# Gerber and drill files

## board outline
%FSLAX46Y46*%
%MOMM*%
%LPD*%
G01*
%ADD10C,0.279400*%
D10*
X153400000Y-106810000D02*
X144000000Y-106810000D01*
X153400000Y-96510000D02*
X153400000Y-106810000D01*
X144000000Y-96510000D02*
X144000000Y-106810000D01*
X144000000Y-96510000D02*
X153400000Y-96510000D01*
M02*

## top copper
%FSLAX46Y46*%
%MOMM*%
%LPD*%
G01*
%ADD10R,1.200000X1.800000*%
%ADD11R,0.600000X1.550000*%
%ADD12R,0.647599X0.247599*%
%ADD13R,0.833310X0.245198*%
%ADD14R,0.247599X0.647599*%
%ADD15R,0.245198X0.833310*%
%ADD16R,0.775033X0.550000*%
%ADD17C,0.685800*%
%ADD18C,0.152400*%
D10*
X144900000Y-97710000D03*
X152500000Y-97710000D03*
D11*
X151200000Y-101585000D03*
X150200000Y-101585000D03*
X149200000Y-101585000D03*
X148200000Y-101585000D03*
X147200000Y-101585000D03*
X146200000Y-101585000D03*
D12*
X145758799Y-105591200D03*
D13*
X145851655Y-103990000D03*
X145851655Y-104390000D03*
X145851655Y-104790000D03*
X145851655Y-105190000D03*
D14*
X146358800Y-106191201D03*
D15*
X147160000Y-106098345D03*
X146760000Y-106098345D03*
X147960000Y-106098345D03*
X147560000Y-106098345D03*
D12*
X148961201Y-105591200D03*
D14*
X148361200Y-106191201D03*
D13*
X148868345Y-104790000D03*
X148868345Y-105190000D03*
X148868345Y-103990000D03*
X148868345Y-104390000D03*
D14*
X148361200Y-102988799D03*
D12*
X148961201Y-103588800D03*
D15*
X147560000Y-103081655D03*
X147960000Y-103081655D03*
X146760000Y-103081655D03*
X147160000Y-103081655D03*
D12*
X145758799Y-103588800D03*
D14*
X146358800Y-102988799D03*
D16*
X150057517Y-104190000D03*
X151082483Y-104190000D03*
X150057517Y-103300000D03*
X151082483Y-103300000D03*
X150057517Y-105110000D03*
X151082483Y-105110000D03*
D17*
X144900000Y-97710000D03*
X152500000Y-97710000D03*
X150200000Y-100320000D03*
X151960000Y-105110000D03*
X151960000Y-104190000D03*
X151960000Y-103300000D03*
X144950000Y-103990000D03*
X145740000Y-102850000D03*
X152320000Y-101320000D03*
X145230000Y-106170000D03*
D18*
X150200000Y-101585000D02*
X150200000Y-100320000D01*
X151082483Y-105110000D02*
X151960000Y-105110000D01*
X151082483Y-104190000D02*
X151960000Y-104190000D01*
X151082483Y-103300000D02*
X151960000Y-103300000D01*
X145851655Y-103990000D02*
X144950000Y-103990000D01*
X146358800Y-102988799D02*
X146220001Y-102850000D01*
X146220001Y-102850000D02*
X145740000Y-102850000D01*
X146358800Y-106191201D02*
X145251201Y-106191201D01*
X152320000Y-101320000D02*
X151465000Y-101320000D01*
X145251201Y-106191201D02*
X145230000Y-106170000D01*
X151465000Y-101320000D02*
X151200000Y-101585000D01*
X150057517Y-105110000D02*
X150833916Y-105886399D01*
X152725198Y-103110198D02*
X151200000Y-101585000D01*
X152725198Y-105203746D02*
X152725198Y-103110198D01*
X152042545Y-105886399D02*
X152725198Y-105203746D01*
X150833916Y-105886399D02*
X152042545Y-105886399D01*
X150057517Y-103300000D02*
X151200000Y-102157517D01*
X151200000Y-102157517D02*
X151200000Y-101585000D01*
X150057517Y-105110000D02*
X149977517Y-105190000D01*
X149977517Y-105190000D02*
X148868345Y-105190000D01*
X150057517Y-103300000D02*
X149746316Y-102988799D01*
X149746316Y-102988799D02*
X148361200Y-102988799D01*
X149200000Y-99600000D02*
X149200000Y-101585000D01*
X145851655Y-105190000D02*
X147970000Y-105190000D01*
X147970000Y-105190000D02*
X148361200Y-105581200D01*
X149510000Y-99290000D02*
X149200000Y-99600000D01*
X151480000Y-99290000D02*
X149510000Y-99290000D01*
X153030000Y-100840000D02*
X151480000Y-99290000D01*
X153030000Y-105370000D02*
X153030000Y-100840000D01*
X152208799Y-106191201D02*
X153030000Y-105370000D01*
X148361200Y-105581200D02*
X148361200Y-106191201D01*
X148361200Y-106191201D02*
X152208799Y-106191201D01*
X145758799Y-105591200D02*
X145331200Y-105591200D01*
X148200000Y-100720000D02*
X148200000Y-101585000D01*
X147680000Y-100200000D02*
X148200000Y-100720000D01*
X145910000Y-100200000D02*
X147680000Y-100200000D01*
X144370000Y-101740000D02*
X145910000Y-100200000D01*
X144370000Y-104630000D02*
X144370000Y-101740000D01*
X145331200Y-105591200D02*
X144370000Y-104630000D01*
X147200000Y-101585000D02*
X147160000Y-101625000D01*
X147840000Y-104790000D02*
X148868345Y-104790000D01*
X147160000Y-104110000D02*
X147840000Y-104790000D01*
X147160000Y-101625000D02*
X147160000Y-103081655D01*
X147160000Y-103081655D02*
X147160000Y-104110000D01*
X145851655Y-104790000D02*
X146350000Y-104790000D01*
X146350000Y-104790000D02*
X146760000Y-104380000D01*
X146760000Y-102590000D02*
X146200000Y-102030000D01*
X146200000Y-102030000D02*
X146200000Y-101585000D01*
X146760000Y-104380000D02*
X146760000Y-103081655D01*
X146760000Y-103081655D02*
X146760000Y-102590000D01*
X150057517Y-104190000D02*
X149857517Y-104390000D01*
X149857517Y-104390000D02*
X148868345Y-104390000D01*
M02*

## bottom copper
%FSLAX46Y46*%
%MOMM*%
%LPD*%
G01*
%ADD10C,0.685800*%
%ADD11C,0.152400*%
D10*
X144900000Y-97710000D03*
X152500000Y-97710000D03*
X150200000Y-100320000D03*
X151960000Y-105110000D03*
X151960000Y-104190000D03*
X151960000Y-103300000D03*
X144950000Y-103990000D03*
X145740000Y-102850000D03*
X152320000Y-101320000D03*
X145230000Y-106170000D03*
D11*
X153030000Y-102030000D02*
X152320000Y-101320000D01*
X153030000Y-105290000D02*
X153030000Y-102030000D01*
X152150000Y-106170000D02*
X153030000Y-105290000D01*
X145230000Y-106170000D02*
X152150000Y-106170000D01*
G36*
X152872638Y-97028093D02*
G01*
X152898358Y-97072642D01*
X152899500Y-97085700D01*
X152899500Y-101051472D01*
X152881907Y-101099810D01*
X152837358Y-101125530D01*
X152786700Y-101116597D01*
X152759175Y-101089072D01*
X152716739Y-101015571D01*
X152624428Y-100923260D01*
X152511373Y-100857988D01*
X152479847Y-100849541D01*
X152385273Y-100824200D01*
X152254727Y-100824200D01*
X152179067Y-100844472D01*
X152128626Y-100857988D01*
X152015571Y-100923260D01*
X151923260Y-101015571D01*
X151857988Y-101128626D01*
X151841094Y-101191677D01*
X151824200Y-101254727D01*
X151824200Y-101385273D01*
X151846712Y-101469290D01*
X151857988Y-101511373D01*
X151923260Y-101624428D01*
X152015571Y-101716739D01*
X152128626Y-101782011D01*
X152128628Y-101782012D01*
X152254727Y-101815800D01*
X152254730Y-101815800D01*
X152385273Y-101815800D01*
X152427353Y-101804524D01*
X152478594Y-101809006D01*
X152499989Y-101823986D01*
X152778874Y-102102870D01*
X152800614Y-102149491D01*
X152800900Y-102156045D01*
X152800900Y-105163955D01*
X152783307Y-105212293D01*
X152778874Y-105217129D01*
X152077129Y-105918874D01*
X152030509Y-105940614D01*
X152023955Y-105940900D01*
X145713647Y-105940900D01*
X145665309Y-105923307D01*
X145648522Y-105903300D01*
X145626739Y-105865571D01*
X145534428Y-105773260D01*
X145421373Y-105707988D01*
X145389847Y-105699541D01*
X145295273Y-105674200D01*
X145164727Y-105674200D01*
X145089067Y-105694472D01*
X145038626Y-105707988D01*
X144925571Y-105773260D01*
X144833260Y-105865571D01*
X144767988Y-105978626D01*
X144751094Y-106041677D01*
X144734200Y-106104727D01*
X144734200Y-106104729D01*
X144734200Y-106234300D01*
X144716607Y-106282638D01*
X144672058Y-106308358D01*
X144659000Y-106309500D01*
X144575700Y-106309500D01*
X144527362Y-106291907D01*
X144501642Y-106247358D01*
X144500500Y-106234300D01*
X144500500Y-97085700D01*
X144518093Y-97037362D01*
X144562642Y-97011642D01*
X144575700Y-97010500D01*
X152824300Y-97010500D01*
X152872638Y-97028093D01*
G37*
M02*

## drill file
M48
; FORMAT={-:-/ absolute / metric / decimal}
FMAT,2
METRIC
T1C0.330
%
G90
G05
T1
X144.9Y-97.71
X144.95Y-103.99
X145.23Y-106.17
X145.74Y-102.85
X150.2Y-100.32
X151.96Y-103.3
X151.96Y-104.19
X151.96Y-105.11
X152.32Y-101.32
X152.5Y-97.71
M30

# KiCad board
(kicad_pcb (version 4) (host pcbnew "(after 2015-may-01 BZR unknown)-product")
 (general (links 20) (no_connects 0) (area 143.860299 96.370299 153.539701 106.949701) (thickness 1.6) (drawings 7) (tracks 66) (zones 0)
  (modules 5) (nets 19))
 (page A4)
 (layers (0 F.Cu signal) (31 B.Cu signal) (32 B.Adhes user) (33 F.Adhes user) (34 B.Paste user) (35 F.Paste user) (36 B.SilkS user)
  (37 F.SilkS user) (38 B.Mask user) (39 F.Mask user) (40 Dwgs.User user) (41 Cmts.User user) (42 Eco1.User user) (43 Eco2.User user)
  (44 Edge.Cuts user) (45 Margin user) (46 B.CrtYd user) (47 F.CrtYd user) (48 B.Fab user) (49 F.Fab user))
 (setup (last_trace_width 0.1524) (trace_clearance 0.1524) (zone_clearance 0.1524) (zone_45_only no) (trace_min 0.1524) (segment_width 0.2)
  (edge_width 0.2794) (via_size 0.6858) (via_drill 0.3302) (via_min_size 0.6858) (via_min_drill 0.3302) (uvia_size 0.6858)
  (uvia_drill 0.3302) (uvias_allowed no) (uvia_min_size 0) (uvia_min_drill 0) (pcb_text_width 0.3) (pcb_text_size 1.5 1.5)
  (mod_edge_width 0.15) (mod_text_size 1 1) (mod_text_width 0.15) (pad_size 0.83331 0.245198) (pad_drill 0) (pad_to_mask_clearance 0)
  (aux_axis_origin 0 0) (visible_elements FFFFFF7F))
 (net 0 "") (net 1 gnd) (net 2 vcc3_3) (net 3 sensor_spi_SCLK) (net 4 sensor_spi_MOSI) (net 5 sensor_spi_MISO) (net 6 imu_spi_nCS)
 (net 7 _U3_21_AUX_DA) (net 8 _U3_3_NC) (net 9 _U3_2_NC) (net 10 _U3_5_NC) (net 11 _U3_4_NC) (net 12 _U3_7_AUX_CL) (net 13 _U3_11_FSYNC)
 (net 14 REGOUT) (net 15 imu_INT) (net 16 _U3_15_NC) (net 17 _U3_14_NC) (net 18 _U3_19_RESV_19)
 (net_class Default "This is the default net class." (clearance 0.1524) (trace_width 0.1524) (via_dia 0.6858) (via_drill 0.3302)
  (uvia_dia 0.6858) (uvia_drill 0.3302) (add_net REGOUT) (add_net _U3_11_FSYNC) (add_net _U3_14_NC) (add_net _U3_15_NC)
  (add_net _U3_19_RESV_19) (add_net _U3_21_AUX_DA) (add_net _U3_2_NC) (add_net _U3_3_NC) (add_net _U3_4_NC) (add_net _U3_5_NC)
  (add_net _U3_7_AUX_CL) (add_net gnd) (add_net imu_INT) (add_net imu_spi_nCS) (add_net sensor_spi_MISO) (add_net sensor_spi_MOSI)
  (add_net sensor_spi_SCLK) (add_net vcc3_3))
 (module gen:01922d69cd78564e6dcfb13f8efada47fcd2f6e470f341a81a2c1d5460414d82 (layer F.Cu) (at 148.7 96.81)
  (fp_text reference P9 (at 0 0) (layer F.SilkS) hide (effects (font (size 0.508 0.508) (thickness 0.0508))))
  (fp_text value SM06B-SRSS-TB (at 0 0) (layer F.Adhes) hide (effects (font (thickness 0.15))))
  (pad M smd rect (at -3.8 0.9) (size 1.2 1.8) (layers F.Cu F.Paste F.Mask) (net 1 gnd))
  (pad M smd rect (at 3.8 0.9) (size 1.2 1.8) (layers F.Cu F.Paste F.Mask) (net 1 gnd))
  (pad 1 smd rect (at 2.5 4.775) (size 0.6 1.55) (layers F.Cu F.Paste F.Mask) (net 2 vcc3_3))
  (pad 2 smd rect (at 1.5 4.775) (size 0.6 1.55) (layers F.Cu F.Paste F.Mask) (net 1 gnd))
  (pad 3 smd rect (at 0.5 4.775) (size 0.6 1.55) (layers F.Cu F.Paste F.Mask) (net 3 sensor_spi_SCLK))
  (pad 4 smd rect (at -0.5 4.775) (size 0.6 1.55) (layers F.Cu F.Paste F.Mask) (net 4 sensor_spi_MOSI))
  (pad 5 smd rect (at -1.5 4.775) (size 0.6 1.55) (layers F.Cu F.Paste F.Mask) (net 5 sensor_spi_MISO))
  (pad 6 smd rect (at -2.5 4.775) (size 0.6 1.55) (layers F.Cu F.Paste F.Mask) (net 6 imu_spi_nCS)))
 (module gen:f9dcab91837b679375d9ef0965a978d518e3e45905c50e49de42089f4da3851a (layer F.Cu) (at 147.36 104.59 90)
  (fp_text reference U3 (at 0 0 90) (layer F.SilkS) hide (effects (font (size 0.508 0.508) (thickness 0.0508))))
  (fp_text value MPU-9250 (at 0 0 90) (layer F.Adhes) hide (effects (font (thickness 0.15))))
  (pad 24 smd rect (at -1.0012 -1.601201 90) (size 0.247599 0.647599) (layers F.Cu F.Paste F.Mask) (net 4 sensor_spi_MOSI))
  (pad 20 smd rect (at 0.6 -1.508345 90) (size 0.245198 0.83331) (layers F.Cu F.Paste F.Mask) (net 1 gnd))
  (pad 21 smd rect (at 0.2 -1.508345 90) (size 0.245198 0.83331) (layers F.Cu F.Paste F.Mask) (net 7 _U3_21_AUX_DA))
  (pad 22 smd rect (at -0.2 -1.508345 90) (size 0.245198 0.83331) (layers F.Cu F.Paste F.Mask) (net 6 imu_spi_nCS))
  (pad 23 smd rect (at -0.6 -1.508345 90) (size 0.245198 0.83331) (layers F.Cu F.Paste F.Mask) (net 3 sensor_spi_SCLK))
  (pad 1 smd rect (at -1.601201 -1.0012 90) (size 0.647599 0.247599) (layers F.Cu F.Paste F.Mask) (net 2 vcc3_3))
  (pad 3 smd rect (at -1.508345 -0.2 90) (size 0.83331 0.245198) (layers F.Cu F.Paste F.Mask) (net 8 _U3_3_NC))
  (pad 2 smd rect (at -1.508345 -0.6 90) (size 0.83331 0.245198) (layers F.Cu F.Paste F.Mask) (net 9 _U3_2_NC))
  (pad 5 smd rect (at -1.508345 0.6 90) (size 0.83331 0.245198) (layers F.Cu F.Paste F.Mask) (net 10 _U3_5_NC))
  (pad 4 smd rect (at -1.508345 0.2 90) (size 0.83331 0.245198) (layers F.Cu F.Paste F.Mask) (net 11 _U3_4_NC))
  (pad 7 smd rect (at -1.0012 1.601201 90) (size 0.247599 0.647599) (layers F.Cu F.Paste F.Mask) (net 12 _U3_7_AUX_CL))
  (pad 6 smd rect (at -1.601201 1.0012 90) (size 0.647599 0.247599) (layers F.Cu F.Paste F.Mask) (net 3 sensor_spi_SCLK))
  (pad 9 smd rect (at -0.2 1.508345 90) (size 0.245198 0.83331) (layers F.Cu F.Paste F.Mask) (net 5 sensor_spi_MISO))
  (pad 8 smd rect (at -0.6 1.508345 90) (size 0.245198 0.83331) (layers F.Cu F.Paste F.Mask) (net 2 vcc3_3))
  (pad 11 smd rect (at 0.6 1.508345 90) (size 0.245198 0.83331) (layers F.Cu F.Paste F.Mask) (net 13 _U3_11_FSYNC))
  (pad 10 smd rect (at 0.2 1.508345 90) (size 0.245198 0.83331) (layers F.Cu F.Paste F.Mask) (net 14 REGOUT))
  (pad 13 smd rect (at 1.601201 1.0012 90) (size 0.647599 0.247599) (layers F.Cu F.Paste F.Mask) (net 2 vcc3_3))
  (pad 12 smd rect (at 1.0012 1.601201 90) (size 0.247599 0.647599) (layers F.Cu F.Paste F.Mask) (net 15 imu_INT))
  (pad 15 smd rect (at 1.508345 0.2 90) (size 0.83331 0.245198) (layers F.Cu F.Paste F.Mask) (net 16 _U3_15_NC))
  (pad 14 smd rect (at 1.508345 0.6 90) (size 0.83331 0.245198) (layers F.Cu F.Paste F.Mask) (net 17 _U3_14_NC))
  (pad 17 smd rect (at 1.508345 -0.6 90) (size 0.83331 0.245198) (layers F.Cu F.Paste F.Mask) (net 6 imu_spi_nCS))
  (pad 16 smd rect (at 1.508345 -0.2 90) (size 0.83331 0.245198) (layers F.Cu F.Paste F.Mask) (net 5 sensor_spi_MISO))
  (pad 19 smd rect (at 1.0012 -1.601201 90) (size 0.247599 0.647599) (layers F.Cu F.Paste F.Mask) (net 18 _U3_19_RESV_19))
  (pad 18 smd rect (at 1.601201 -1.0012 90) (size 0.647599 0.247599) (layers F.Cu F.Paste F.Mask) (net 1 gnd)))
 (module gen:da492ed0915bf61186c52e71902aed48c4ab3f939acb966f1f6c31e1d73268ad (layer F.Cu) (at 150.57 104.19)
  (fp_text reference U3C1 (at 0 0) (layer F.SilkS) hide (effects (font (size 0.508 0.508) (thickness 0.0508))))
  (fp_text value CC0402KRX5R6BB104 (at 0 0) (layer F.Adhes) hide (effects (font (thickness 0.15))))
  (pad 1 smd rect (at -0.512483 0) (size 0.775033 0.55) (layers F.Cu F.Paste F.Mask) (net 14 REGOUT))
  (pad 2 smd rect (at 0.512483 0) (size 0.775033 0.55) (layers F.Cu F.Paste F.Mask) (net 1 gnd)))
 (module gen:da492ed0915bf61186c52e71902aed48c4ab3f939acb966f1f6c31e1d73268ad (layer F.Cu) (at 150.57 103.3)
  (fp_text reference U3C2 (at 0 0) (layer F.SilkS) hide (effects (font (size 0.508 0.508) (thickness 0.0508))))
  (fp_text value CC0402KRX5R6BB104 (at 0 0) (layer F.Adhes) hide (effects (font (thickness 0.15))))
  (pad 1 smd rect (at -0.512483 0) (size 0.775033 0.55) (layers F.Cu F.Paste F.Mask) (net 2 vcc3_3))
  (pad 2 smd rect (at 0.512483 0) (size 0.775033 0.55) (layers F.Cu F.Paste F.Mask) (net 1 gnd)))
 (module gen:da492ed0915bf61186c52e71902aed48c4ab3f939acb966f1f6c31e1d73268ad (layer F.Cu) (at 150.57 105.11)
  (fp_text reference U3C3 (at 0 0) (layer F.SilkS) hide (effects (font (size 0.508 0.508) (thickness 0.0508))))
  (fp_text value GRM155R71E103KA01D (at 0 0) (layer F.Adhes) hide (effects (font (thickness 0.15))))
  (pad 1 smd rect (at -0.512483 0) (size 0.775033 0.55) (layers F.Cu F.Paste F.Mask) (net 2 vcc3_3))
  (pad 2 smd rect (at 0.512483 0) (size 0.775033 0.55) (layers F.Cu F.Paste F.Mask) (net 1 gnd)))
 (gr_line (start 153.4 106.81) (end 144 106.81) (angle 90) (layer Edge.Cuts) (width 0.2794))
 (gr_line (start 153.4 96.51) (end 153.4 106.81) (angle 90) (layer Edge.Cuts) (width 0.2794))
 (gr_line (start 144 96.51) (end 144 106.81) (angle 90) (layer Edge.Cuts) (width 0.2794))
 (gr_line (start 144 96.51) (end 153.4 96.51) (angle 90) (layer Edge.Cuts) (width 0.2794))
 (via (at 144.9 97.71) (size 0.6858) (layers F.Cu B.Cu) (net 1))
 (via (at 152.5 97.71) (size 0.6858) (layers F.Cu B.Cu) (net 1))
 (segment (start 150.2 101.585) (end 150.2 100.32) (width 0.1524) (layer F.Cu) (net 1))
 (via (at 150.2 100.32) (size 0.6858) (layers F.Cu B.Cu) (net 1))
 (segment (start 151.082483 105.11) (end 151.96 105.11) (width 0.1524) (layer F.Cu) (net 1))
 (via (at 151.96 105.11) (size 0.6858) (layers F.Cu B.Cu) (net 1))
 (segment (start 151.082483 104.19) (end 151.96 104.19) (width 0.1524) (layer F.Cu) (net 1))
 (via (at 151.96 104.19) (size 0.6858) (layers F.Cu B.Cu) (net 1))
 (segment (start 151.082483 103.3) (end 151.96 103.3) (width 0.1524) (layer F.Cu) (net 1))
 (via (at 151.96 103.3) (size 0.6858) (layers F.Cu B.Cu) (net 1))
 (segment (start 145.851655 103.99) (end 144.95 103.99) (width 0.1524) (layer F.Cu) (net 1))
 (via (at 144.95 103.99) (size 0.6858) (layers F.Cu B.Cu) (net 1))
 (segment (start 146.3588 102.988799) (end 146.220001 102.85) (width 0.1524) (layer F.Cu) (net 1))
 (via (at 145.74 102.85) (size 0.6858) (layers F.Cu B.Cu) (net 1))
 (segment (start 146.220001 102.85) (end 145.74 102.85) (width 0.1524) (layer F.Cu) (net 1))
 (segment (start 146.3588 106.191201) (end 145.251201 106.191201) (width 0.1524) (layer F.Cu) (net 2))
 (segment (start 152.32 101.32) (end 151.465 101.32) (width 0.1524) (layer F.Cu) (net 2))
 (via (at 152.32 101.32) (size 0.6858) (layers F.Cu B.Cu) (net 2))
 (segment (start 153.03 102.03) (end 152.32 101.32) (width 0.1524) (layer B.Cu) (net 2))
 (segment (start 153.03 105.29) (end 153.03 102.03) (width 0.1524) (layer B.Cu) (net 2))
 (segment (start 152.15 106.17) (end 153.03 105.29) (width 0.1524) (layer B.Cu) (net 2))
 (segment (start 145.23 106.17) (end 152.15 106.17) (width 0.1524) (layer B.Cu) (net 2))
 (via (at 145.23 106.17) (size 0.6858) (layers F.Cu B.Cu) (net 2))
 (segment (start 145.251201 106.191201) (end 145.23 106.17) (width 0.1524) (layer F.Cu) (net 2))
 (segment (start 151.465 101.32) (end 151.2 101.585) (width 0.1524) (layer F.Cu) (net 2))
 (segment (start 150.057517 105.11) (end 150.833916 105.886399) (width 0.1524) (layer F.Cu) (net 2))
 (segment (start 152.725198 103.110198) (end 151.2 101.585) (width 0.1524) (layer F.Cu) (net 2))
 (segment (start 152.725198 105.203746) (end 152.725198 103.110198) (width 0.1524) (layer F.Cu) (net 2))
 (segment (start 152.042545 105.886399) (end 152.725198 105.203746) (width 0.1524) (layer F.Cu) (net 2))
 (segment (start 150.833916 105.886399) (end 152.042545 105.886399) (width 0.1524) (layer F.Cu) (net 2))
 (segment (start 150.057517 103.3) (end 151.2 102.157517) (width 0.1524) (layer F.Cu) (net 2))
 (segment (start 151.2 102.157517) (end 151.2 101.585) (width 0.1524) (layer F.Cu) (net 2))
 (segment (start 150.057517 105.11) (end 149.977517 105.19) (width 0.1524) (layer F.Cu) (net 2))
 (segment (start 149.977517 105.19) (end 148.868345 105.19) (width 0.1524) (layer F.Cu) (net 2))
 (segment (start 150.057517 103.3) (end 149.746316 102.988799) (width 0.1524) (layer F.Cu) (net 2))
 (segment (start 149.746316 102.988799) (end 148.3612 102.988799) (width 0.1524) (layer F.Cu) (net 2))
 (segment (start 149.2 99.6) (end 149.2 101.585) (width 0.1524) (layer F.Cu) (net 3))
 (segment (start 145.851655 105.19) (end 147.97 105.19) (width 0.1524) (layer F.Cu) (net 3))
 (segment (start 147.97 105.19) (end 148.3612 105.5812) (width 0.1524) (layer F.Cu) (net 3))
 (segment (start 149.51 99.29) (end 149.2 99.6) (width 0.1524) (layer F.Cu) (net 3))
 (segment (start 151.48 99.29) (end 149.51 99.29) (width 0.1524) (layer F.Cu) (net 3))
 (segment (start 153.03 100.84) (end 151.48 99.29) (width 0.1524) (layer F.Cu) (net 3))
 (segment (start 153.03 105.37) (end 153.03 100.84) (width 0.1524) (layer F.Cu) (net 3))
 (segment (start 152.208799 106.191201) (end 153.03 105.37) (width 0.1524) (layer F.Cu) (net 3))
 (segment (start 148.3612 105.5812) (end 148.3612 106.191201) (width 0.1524) (layer F.Cu) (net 3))
 (segment (start 148.3612 106.191201) (end 152.208799 106.191201) (width 0.1524) (layer F.Cu) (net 3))
 (segment (start 145.758799 105.5912) (end 145.3312 105.5912) (width 0.1524) (layer F.Cu) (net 4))
 (segment (start 148.2 100.72) (end 148.2 101.585) (width 0.1524) (layer F.Cu) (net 4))
 (segment (start 147.68 100.2) (end 148.2 100.72) (width 0.1524) (layer F.Cu) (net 4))
 (segment (start 145.91 100.2) (end 147.68 100.2) (width 0.1524) (layer F.Cu) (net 4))
 (segment (start 144.37 101.74) (end 145.91 100.2) (width 0.1524) (layer F.Cu) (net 4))
 (segment (start 144.37 104.63) (end 144.37 101.74) (width 0.1524) (layer F.Cu) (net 4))
 (segment (start 145.3312 105.5912) (end 144.37 104.63) (width 0.1524) (layer F.Cu) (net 4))
 (segment (start 147.2 101.585) (end 147.16 101.625) (width 0.1524) (layer F.Cu) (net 5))
 (segment (start 147.84 104.79) (end 148.868345 104.79) (width 0.1524) (layer F.Cu) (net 5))
 (segment (start 147.16 104.11) (end 147.84 104.79) (width 0.1524) (layer F.Cu) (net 5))
 (segment (start 147.16 101.625) (end 147.16 103.081655) (width 0.1524) (layer F.Cu) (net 5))
 (segment (start 147.16 103.081655) (end 147.16 104.11) (width 0.1524) (layer F.Cu) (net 5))
 (segment (start 145.851655 104.79) (end 146.35 104.79) (width 0.1524) (layer F.Cu) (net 6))
 (segment (start 146.35 104.79) (end 146.76 104.38) (width 0.1524) (layer F.Cu) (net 6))
 (segment (start 146.76 102.59) (end 146.2 102.03) (width 0.1524) (layer F.Cu) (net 6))
 (segment (start 146.2 102.03) (end 146.2 101.585) (width 0.1524) (layer F.Cu) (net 6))
 (segment (start 146.76 104.38) (end 146.76 103.081655) (width 0.1524) (layer F.Cu) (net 6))
 (segment (start 146.76 103.081655) (end 146.76 102.59) (width 0.1524) (layer F.Cu) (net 6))
 (segment (start 150.057517 104.19) (end 149.857517 104.39) (width 0.1524) (layer F.Cu) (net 14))
 (segment (start 149.857517 104.39) (end 148.868345 104.39) (width 0.1524) (layer F.Cu) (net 14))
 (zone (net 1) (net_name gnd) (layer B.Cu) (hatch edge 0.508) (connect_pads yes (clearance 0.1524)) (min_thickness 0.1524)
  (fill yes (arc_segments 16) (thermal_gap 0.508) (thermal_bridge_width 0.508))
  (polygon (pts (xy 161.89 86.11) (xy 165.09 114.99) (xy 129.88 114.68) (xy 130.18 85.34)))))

